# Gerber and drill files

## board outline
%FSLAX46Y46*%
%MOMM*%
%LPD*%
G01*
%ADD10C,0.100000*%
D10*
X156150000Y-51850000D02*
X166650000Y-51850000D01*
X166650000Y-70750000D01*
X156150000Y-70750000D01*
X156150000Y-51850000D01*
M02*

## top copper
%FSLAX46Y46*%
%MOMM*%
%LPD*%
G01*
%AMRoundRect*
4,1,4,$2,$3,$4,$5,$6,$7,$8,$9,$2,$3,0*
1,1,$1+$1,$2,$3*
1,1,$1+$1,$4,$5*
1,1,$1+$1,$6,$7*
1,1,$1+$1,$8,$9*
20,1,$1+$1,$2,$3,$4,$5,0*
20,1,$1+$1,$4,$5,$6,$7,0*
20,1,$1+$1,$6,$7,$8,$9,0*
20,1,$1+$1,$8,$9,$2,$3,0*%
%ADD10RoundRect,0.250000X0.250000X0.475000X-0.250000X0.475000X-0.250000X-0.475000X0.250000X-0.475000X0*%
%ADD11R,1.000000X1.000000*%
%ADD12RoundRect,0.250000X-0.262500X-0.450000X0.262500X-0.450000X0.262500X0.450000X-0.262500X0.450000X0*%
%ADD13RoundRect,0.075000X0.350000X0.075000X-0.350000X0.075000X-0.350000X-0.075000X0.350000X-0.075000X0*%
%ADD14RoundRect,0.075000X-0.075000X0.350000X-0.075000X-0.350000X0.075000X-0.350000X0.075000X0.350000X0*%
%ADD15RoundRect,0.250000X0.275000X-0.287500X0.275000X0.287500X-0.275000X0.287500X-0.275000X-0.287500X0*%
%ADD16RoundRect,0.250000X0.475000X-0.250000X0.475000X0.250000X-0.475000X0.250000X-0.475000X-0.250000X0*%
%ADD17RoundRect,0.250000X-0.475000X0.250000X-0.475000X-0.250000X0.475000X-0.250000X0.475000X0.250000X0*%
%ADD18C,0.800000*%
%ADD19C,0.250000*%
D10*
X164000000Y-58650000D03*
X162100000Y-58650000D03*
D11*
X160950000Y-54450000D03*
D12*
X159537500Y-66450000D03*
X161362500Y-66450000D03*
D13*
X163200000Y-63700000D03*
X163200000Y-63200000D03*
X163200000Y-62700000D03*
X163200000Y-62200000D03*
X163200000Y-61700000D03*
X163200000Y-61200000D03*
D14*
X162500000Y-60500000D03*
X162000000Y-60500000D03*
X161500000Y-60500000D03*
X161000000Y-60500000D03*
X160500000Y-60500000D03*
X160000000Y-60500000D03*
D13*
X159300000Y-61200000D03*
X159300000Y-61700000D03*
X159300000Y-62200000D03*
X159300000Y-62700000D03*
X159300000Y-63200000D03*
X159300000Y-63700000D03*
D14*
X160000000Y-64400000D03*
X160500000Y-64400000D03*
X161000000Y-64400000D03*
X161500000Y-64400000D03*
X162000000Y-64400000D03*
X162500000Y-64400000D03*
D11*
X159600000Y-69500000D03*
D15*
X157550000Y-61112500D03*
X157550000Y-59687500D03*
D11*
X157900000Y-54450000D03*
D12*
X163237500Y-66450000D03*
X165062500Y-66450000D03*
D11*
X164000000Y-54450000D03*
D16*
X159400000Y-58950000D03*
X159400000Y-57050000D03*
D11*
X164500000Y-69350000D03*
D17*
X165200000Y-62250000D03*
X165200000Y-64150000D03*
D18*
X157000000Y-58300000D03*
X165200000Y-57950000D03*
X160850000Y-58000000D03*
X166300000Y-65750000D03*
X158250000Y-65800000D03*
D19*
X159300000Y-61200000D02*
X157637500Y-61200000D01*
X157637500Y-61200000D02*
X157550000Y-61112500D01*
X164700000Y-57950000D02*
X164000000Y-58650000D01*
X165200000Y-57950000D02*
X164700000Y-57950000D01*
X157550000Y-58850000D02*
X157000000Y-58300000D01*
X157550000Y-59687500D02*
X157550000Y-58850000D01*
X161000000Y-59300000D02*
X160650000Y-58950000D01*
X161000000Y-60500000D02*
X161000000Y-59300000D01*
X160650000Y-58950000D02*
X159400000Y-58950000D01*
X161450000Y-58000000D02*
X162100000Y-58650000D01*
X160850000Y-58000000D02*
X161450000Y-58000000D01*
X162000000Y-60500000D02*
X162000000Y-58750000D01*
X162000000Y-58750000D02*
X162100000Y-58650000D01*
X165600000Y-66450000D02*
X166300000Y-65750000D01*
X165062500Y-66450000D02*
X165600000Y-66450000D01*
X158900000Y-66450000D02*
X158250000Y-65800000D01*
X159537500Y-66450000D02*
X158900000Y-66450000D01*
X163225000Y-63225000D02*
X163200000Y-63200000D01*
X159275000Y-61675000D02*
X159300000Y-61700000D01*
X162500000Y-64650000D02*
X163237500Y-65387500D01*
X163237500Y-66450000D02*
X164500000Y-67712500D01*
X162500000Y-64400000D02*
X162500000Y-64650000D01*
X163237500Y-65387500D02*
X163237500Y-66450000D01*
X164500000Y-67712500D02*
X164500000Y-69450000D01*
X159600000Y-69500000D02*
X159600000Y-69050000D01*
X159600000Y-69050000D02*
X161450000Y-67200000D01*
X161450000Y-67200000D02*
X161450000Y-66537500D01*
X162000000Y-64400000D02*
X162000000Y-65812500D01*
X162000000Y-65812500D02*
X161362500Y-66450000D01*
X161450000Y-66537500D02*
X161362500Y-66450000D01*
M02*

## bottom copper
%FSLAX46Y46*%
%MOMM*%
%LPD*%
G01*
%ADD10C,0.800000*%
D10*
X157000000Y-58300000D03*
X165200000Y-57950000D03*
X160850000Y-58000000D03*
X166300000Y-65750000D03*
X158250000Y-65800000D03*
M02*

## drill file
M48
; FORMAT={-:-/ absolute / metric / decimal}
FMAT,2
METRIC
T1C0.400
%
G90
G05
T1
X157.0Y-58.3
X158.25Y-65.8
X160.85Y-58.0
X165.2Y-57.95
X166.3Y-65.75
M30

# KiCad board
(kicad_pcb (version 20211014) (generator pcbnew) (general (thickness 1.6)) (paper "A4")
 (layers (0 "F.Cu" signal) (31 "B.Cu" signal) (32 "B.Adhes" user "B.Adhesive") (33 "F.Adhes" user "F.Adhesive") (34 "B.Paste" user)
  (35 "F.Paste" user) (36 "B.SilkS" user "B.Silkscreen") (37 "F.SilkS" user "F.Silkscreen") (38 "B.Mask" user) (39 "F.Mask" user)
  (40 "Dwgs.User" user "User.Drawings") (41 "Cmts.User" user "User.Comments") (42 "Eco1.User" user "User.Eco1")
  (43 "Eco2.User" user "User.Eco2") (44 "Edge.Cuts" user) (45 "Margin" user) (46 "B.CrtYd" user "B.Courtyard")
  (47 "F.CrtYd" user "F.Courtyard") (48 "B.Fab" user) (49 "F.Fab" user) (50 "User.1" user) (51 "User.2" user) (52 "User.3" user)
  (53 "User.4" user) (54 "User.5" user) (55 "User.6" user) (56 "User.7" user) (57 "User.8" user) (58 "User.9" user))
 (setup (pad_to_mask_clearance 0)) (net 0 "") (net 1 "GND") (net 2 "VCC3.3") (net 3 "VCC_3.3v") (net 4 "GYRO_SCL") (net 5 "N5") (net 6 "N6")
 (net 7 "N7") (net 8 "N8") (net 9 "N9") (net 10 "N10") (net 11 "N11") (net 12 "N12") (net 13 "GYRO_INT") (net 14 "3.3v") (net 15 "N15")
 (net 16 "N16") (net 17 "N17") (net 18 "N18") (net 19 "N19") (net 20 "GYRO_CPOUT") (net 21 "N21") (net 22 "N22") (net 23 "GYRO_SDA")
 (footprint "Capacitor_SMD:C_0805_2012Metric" (layer "F.Cu") (at 163.05 58.65 180)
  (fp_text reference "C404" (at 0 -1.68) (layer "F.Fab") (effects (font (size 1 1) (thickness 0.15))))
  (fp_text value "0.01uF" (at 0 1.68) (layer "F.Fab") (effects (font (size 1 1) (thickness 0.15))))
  (pad "1" smd roundrect (at -0.95 0 180) (size 1 1.45) (layers "F.Cu" "F.Paste" "F.Mask") (roundrect_rratio 0.25) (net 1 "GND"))
  (pad "2" smd roundrect (at 0.95 0 180) (size 1 1.45) (layers "F.Cu" "F.Paste" "F.Mask") (roundrect_rratio 0.25) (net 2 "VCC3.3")))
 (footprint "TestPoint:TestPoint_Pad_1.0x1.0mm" (layer "F.Cu") (at 160.95 54.45)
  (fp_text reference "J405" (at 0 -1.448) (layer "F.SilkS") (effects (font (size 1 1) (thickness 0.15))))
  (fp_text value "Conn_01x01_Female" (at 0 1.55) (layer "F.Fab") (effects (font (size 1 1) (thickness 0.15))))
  (pad "1" smd rect (at 0 0) (size 1 1) (layers "F.Cu" "F.Mask") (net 2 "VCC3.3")))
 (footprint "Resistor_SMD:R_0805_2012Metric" (layer "F.Cu") (at 160.45 66.45)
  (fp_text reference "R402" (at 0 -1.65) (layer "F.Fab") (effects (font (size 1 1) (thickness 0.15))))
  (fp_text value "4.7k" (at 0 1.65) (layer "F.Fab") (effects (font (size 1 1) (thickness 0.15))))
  (pad "1" smd roundrect (at -0.9125 0) (size 1.025 1.4) (layers "F.Cu" "F.Paste" "F.Mask") (roundrect_rratio 0.243902) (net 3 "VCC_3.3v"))
  (pad "2" smd roundrect (at 0.9125 0) (size 1.025 1.4) (layers "F.Cu" "F.Paste" "F.Mask") (roundrect_rratio 0.243902) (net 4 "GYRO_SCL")))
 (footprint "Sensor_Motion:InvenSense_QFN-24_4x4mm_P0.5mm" (layer "F.Cu") (at 161.25 62.45 180)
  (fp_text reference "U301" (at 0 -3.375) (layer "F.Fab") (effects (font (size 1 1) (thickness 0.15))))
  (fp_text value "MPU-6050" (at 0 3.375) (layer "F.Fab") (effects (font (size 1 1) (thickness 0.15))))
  (pad "1" smd roundrect (at -1.95 -1.25 180) (size 0.85 0.3) (layers "F.Cu" "F.Paste" "F.Mask") (roundrect_rratio 0.25) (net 1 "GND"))
  (pad "2" smd roundrect (at -1.95 -0.75 180) (size 0.85 0.3) (layers "F.Cu" "F.Paste" "F.Mask") (roundrect_rratio 0.25) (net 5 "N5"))
  (pad "3" smd roundrect (at -1.95 -0.25 180) (size 0.85 0.3) (layers "F.Cu" "F.Paste" "F.Mask") (roundrect_rratio 0.25) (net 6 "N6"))
  (pad "4" smd roundrect (at -1.95 0.25 180) (size 0.85 0.3) (layers "F.Cu" "F.Paste" "F.Mask") (roundrect_rratio 0.25) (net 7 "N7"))
  (pad "5" smd roundrect (at -1.95 0.75 180) (size 0.85 0.3) (layers "F.Cu" "F.Paste" "F.Mask") (roundrect_rratio 0.25) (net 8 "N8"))
  (pad "6" smd roundrect (at -1.95 1.25 180) (size 0.85 0.3) (layers "F.Cu" "F.Paste" "F.Mask") (roundrect_rratio 0.25) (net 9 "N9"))
  (pad "7" smd roundrect (at -1.25 1.95 270) (size 0.85 0.3) (layers "F.Cu" "F.Paste" "F.Mask") (roundrect_rratio 0.25) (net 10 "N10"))
  (pad "8" smd roundrect (at -0.75 1.95 270) (size 0.85 0.3) (layers "F.Cu" "F.Paste" "F.Mask") (roundrect_rratio 0.25) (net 2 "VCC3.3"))
  (pad "9" smd roundrect (at -0.25 1.95 270) (size 0.85 0.3) (layers "F.Cu" "F.Paste" "F.Mask") (roundrect_rratio 0.25) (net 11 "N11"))
  (pad "10" smd roundrect (at 0.25 1.95 270) (size 0.85 0.3) (layers "F.Cu" "F.Paste" "F.Mask") (roundrect_rratio 0.25) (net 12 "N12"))
  (pad "11" smd roundrect (at 0.75 1.95 270) (size 0.85 0.3) (layers "F.Cu" "F.Paste" "F.Mask") (roundrect_rratio 0.25) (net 1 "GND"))
  (pad "12" smd roundrect (at 1.25 1.95 270) (size 0.85 0.3) (layers "F.Cu" "F.Paste" "F.Mask") (roundrect_rratio 0.25) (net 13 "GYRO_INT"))
  (pad "13" smd roundrect (at 1.95 1.25 180) (size 0.85 0.3) (layers "F.Cu" "F.Paste" "F.Mask") (roundrect_rratio 0.25) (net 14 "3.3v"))
  (pad "14" smd roundrect (at 1.95 0.75 180) (size 0.85 0.3) (layers "F.Cu" "F.Paste" "F.Mask") (roundrect_rratio 0.25) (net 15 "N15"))
  (pad "15" smd roundrect (at 1.95 0.25 180) (size 0.85 0.3) (layers "F.Cu" "F.Paste" "F.Mask") (roundrect_rratio 0.25) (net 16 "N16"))
  (pad "16" smd roundrect (at 1.95 -0.25 180) (size 0.85 0.3) (layers "F.Cu" "F.Paste" "F.Mask") (roundrect_rratio 0.25) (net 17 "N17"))
  (pad "17" smd roundrect (at 1.95 -0.75 180) (size 0.85 0.3) (layers "F.Cu" "F.Paste" "F.Mask") (roundrect_rratio 0.25) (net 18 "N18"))
  (pad "18" smd roundrect (at 1.95 -1.25 180) (size 0.85 0.3) (layers "F.Cu" "F.Paste" "F.Mask") (roundrect_rratio 0.25) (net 1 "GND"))
  (pad "19" smd roundrect (at 1.25 -1.95 270) (size 0.85 0.3) (layers "F.Cu" "F.Paste" "F.Mask") (roundrect_rratio 0.25) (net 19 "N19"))
  (pad "20" smd roundrect (at 0.75 -1.95 270) (size 0.85 0.3) (layers "F.Cu" "F.Paste" "F.Mask") (roundrect_rratio 0.25)
   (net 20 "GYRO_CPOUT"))
  (pad "21" smd roundrect (at 0.25 -1.95 270) (size 0.85 0.3) (layers "F.Cu" "F.Paste" "F.Mask") (roundrect_rratio 0.25) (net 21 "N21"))
  (pad "22" smd roundrect (at -0.25 -1.95 270) (size 0.85 0.3) (layers "F.Cu" "F.Paste" "F.Mask") (roundrect_rratio 0.25) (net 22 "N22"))
  (pad "23" smd roundrect (at -0.75 -1.95 270) (size 0.85 0.3) (layers "F.Cu" "F.Paste" "F.Mask") (roundrect_rratio 0.25) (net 4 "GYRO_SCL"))
  (pad "24" smd roundrect (at -1.25 -1.95 270) (size 0.85 0.3) (layers "F.Cu" "F.Paste" "F.Mask") (roundrect_rratio 0.25)
   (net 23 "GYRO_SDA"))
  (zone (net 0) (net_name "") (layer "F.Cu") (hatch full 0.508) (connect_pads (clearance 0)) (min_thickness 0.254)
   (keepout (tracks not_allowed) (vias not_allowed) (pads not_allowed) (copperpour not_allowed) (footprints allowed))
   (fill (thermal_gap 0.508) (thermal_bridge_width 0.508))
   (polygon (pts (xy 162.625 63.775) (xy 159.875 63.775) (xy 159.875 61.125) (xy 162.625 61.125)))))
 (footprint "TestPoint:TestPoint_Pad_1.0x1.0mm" (layer "F.Cu") (at 159.6 69.5 180)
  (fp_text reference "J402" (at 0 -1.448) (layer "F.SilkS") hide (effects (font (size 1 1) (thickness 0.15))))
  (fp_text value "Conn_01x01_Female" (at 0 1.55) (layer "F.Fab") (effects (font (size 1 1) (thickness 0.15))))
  (pad "1" smd rect (at 0 0 180) (size 1 1) (layers "F.Cu" "F.Mask") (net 4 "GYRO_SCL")))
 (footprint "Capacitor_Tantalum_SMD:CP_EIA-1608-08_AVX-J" (layer "F.Cu") (at 157.55 60.4 90)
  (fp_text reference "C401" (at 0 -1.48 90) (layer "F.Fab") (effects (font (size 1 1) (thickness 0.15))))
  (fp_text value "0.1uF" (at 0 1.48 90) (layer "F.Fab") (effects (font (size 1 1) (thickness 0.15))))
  (pad "1" smd roundrect (at -0.7125 0 90) (size 1.075 1.05) (layers "F.Cu" "F.Paste" "F.Mask") (roundrect_rratio 0.238095) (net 14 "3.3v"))
  (pad "2" smd roundrect (at 0.7125 0 90) (size 1.075 1.05) (layers "F.Cu" "F.Paste" "F.Mask") (roundrect_rratio 0.238095) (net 1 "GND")))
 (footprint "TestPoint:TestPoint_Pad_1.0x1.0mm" (layer "F.Cu") (at 157.9 54.45)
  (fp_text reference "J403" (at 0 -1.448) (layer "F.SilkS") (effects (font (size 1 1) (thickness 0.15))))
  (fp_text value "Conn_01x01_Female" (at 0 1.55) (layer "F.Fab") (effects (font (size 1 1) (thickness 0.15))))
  (pad "1" smd rect (at 0 0) (size 1 1) (layers "F.Cu" "F.Mask") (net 13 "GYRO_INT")))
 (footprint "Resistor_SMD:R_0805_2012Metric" (layer "F.Cu") (at 164.15 66.45)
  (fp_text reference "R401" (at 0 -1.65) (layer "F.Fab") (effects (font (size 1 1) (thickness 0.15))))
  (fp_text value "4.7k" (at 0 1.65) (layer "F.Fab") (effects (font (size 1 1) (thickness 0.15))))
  (pad "1" smd roundrect (at -0.9125 0) (size 1.025 1.4) (layers "F.Cu" "F.Paste" "F.Mask") (roundrect_rratio 0.243902) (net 23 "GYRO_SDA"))
  (pad "2" smd roundrect (at 0.9125 0) (size 1.025 1.4) (layers "F.Cu" "F.Paste" "F.Mask") (roundrect_rratio 0.243902) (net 3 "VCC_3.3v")))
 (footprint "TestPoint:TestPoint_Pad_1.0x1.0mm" (layer "F.Cu") (at 164 54.45)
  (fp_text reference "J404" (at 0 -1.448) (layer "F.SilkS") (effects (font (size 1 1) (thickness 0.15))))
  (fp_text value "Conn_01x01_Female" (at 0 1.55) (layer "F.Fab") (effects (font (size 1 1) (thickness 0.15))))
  (pad "1" smd rect (at 0 0) (size 1 1) (layers "F.Cu" "F.Mask") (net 1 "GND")))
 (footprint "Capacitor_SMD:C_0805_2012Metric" (layer "F.Cu") (at 159.4 58 90)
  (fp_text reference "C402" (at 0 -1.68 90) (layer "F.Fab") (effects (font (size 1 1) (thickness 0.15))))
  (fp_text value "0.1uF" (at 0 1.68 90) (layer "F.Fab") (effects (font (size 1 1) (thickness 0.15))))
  (pad "1" smd roundrect (at -0.95 0 90) (size 1 1.45) (layers "F.Cu" "F.Paste" "F.Mask") (roundrect_rratio 0.25) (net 12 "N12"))
  (pad "2" smd roundrect (at 0.95 0 90) (size 1 1.45) (layers "F.Cu" "F.Paste" "F.Mask") (roundrect_rratio 0.25) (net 1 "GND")))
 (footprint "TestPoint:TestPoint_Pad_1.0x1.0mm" (layer "F.Cu") (at 164.5 69.35 180)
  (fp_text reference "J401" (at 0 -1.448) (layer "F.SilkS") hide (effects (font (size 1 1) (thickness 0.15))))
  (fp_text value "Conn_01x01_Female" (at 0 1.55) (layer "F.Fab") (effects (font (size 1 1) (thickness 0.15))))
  (pad "1" smd rect (at 0 0 180) (size 1 1) (layers "F.Cu" "F.Mask") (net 23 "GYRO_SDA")))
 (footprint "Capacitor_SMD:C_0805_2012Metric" (layer "F.Cu") (at 165.2 63.2 -90)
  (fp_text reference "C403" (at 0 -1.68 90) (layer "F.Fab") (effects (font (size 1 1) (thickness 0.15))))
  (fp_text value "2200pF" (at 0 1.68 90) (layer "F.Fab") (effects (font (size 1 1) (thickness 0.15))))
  (pad "1" smd roundrect (at -0.95 0 270) (size 1 1.45) (layers "F.Cu" "F.Paste" "F.Mask") (roundrect_rratio 0.25) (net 1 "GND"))
  (pad "2" smd roundrect (at 0.95 0 270) (size 1 1.45) (layers "F.Cu" "F.Paste" "F.Mask") (roundrect_rratio 0.25) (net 20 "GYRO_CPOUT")))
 (gr_rect (start 156.15 70.75) (end 166.65 51.85) (layer "Edge.Cuts") (width 0.1) (fill none))
 (segment (start 159.3 61.2) (end 157.6375 61.2) (width 0.25) (layer "F.Cu") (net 14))
 (segment (start 157.6375 61.2) (end 157.55 61.1125) (width 0.25) (layer "F.Cu") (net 14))
 (segment (start 164.7 57.95) (end 164 58.65) (width 0.25) (layer "F.Cu") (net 1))
 (segment (start 165.2 57.95) (end 164.7 57.95) (width 0.25) (layer "F.Cu") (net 1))
 (segment (start 157.55 58.85) (end 157 58.3) (width 0.25) (layer "F.Cu") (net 1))
 (segment (start 157.55 59.6875) (end 157.55 58.85) (width 0.25) (layer "F.Cu") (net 1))
 (via (at 157 58.3) (size 0.8) (drill 0.4) (layers "F.Cu" "B.Cu") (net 1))
 (via (at 165.2 57.95) (size 0.8) (drill 0.4) (layers "F.Cu" "B.Cu") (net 1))
 (segment (start 161 59.3) (end 160.65 58.95) (width 0.25) (layer "F.Cu") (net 12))
 (segment (start 161 60.5) (end 161 59.3) (width 0.25) (layer "F.Cu") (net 12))
 (segment (start 160.65 58.95) (end 159.4 58.95) (width 0.25) (layer "F.Cu") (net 12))
 (segment (start 161.45 58) (end 162.1 58.65) (width 0.25) (layer "F.Cu") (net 2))
 (segment (start 160.85 58) (end 161.45 58) (width 0.25) (layer "F.Cu") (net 2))
 (segment (start 162 60.5) (end 162 58.75) (width 0.25) (layer "F.Cu") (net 2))
 (segment (start 162 58.75) (end 162.1 58.65) (width 0.25) (layer "F.Cu") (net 2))
 (via (at 160.85 58) (size 0.8) (drill 0.4) (layers "F.Cu" "B.Cu") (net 2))
 (segment (start 165.6 66.45) (end 166.3 65.75) (width 0.25) (layer "F.Cu") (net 3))
 (segment (start 165.0625 66.45) (end 165.6 66.45) (width 0.25) (layer "F.Cu") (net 3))
 (segment (start 158.9 66.45) (end 158.25 65.8) (width 0.25) (layer "F.Cu") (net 3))
 (segment (start 159.5375 66.45) (end 158.9 66.45) (width 0.25) (layer "F.Cu") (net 3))
 (via (at 166.3 65.75) (size 0.8) (drill 0.4) (layers "F.Cu" "B.Cu") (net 3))
 (via (at 158.25 65.8) (size 0.8) (drill 0.4) (layers "F.Cu" "B.Cu") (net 3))
 (segment (start 163.225 63.225) (end 163.2 63.2) (width 0.25) (layer "F.Cu") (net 5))
 (segment (start 159.275 61.675) (end 159.3 61.7) (width 0.25) (layer "F.Cu") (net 15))
 (segment (start 162.5 64.65) (end 163.2375 65.3875) (width 0.25) (layer "F.Cu") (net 23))
 (segment (start 163.2375 66.45) (end 164.5 67.7125) (width 0.25) (layer "F.Cu") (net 23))
 (segment (start 162.5 64.4) (end 162.5 64.65) (width 0.25) (layer "F.Cu") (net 23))
 (segment (start 163.2375 65.3875) (end 163.2375 66.45) (width 0.25) (layer "F.Cu") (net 23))
 (segment (start 164.5 67.7125) (end 164.5 69.45) (width 0.25) (layer "F.Cu") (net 23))
 (segment (start 159.6 69.5) (end 159.6 69.05) (width 0.25) (layer "F.Cu") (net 4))
 (segment (start 159.6 69.05) (end 161.45 67.2) (width 0.25) (layer "F.Cu") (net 4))
 (segment (start 161.45 67.2) (end 161.45 66.5375) (width 0.25) (layer "F.Cu") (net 4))
 (segment (start 162 64.4) (end 162 65.8125) (width 0.25) (layer "F.Cu") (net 4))
 (segment (start 162 65.8125) (end 161.3625 66.45) (width 0.25) (layer "F.Cu") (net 4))
 (segment (start 161.45 66.5375) (end 161.3625 66.45) (width 0.25) (layer "F.Cu") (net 4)))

